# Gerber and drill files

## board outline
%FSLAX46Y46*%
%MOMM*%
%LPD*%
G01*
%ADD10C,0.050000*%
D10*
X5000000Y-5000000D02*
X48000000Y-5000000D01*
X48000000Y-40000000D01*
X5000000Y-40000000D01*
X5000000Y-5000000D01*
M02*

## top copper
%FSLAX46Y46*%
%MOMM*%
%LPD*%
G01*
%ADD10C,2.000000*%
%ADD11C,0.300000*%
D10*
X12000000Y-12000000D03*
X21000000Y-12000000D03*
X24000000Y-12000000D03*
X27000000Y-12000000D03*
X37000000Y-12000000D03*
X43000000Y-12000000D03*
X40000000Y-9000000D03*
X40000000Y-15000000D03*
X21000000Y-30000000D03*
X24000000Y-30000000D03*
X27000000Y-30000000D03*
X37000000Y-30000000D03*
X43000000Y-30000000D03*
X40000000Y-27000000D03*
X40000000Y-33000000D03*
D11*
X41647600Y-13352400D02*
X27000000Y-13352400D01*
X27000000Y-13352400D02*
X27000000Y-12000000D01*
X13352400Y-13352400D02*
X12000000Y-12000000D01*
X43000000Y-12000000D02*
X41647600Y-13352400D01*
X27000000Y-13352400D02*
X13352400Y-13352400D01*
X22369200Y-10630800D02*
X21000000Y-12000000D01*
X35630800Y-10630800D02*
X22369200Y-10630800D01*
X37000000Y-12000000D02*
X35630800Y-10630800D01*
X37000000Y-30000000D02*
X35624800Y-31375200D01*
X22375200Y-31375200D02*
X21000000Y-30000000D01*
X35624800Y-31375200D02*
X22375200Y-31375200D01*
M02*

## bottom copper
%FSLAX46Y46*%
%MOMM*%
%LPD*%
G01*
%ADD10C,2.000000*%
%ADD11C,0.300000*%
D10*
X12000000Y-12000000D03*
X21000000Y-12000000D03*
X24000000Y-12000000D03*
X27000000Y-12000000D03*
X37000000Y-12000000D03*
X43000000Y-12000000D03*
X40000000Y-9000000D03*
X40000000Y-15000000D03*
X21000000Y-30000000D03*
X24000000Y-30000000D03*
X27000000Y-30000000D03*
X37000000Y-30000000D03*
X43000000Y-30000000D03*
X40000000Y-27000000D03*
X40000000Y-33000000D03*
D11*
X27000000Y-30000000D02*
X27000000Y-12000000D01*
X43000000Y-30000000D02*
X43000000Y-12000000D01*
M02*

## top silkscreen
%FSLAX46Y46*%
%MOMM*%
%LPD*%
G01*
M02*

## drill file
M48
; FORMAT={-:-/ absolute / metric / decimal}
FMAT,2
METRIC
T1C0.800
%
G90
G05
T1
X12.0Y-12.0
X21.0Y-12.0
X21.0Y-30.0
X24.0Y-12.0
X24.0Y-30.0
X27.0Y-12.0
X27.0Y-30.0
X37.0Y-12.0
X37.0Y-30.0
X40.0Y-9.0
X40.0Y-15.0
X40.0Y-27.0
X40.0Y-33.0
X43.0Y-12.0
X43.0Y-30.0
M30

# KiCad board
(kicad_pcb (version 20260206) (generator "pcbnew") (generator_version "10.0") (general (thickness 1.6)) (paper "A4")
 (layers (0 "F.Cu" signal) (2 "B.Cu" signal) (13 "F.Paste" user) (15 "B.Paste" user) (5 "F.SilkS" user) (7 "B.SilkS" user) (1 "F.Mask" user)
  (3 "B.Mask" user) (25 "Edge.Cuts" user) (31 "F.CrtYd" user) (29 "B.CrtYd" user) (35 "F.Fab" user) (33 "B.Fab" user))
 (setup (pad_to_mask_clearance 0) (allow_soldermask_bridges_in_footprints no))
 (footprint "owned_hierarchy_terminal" (layer "F.Cu") (at 12 12)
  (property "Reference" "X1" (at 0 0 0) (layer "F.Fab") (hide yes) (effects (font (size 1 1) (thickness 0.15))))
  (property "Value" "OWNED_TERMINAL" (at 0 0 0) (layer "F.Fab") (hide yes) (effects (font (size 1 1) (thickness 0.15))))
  (pad "1" thru_hole circle (at 0 0) (size 2 2) (drill 0.8) (layers "*.Cu" "*.Mask") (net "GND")))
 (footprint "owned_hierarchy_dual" (layer "F.Cu") (at 24 12)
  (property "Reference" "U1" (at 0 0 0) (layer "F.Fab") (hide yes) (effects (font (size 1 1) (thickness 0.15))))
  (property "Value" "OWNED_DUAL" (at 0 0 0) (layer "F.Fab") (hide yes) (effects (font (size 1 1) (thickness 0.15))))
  (pad "1" thru_hole circle (at -3 0) (size 2 2) (drill 0.8) (layers "*.Cu" "*.Mask") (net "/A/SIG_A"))
  (pad "2" thru_hole circle (at 0 0) (size 2 2) (drill 0.8) (layers "*.Cu" "*.Mask") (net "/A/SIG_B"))
  (pad "3" thru_hole circle (at 3 0) (size 2 2) (drill 0.8) (layers "*.Cu" "*.Mask") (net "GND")))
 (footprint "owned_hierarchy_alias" (layer "F.Cu") (at 40 12)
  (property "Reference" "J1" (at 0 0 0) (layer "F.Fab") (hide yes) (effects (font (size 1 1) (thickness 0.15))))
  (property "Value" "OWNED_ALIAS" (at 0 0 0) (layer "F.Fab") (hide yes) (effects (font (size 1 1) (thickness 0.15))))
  (pad "R" thru_hole circle (at -3 0) (size 2 2) (drill 0.8) (layers "*.Cu" "*.Mask") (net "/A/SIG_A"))
  (pad "T" thru_hole circle (at 3 0) (size 2 2) (drill 0.8) (layers "*.Cu" "*.Mask") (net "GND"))
  (pad "MP" thru_hole circle (at 0 -3) (size 2 2) (drill 0.8) (layers "*.Cu" "*.Mask"))
  (pad "MP" thru_hole circle (at 0 3) (size 2 2) (drill 0.8) (layers "*.Cu" "*.Mask")))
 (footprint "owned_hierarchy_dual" (layer "F.Cu") (at 24 30)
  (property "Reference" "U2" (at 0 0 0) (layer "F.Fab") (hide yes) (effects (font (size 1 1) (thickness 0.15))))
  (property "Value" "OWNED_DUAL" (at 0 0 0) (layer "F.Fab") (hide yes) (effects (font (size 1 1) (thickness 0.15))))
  (pad "1" thru_hole circle (at -3 0) (size 2 2) (drill 0.8) (layers "*.Cu" "*.Mask") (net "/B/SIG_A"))
  (pad "2" thru_hole circle (at 0 0) (size 2 2) (drill 0.8) (layers "*.Cu" "*.Mask") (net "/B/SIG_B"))
  (pad "3" thru_hole circle (at 3 0) (size 2 2) (drill 0.8) (layers "*.Cu" "*.Mask") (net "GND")))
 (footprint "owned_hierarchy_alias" (layer "F.Cu") (at 40 30)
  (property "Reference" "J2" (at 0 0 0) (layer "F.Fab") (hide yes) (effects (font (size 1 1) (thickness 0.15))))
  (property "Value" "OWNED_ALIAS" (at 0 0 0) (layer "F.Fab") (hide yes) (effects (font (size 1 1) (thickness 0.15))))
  (pad "R" thru_hole circle (at -3 0) (size 2 2) (drill 0.8) (layers "*.Cu" "*.Mask") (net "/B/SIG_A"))
  (pad "T" thru_hole circle (at 3 0) (size 2 2) (drill 0.8) (layers "*.Cu" "*.Mask") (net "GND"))
  (pad "MP" thru_hole circle (at 0 -3) (size 2 2) (drill 0.8) (layers "*.Cu" "*.Mask"))
  (pad "MP" thru_hole circle (at 0 3) (size 2 2) (drill 0.8) (layers "*.Cu" "*.Mask")))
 (gr_rect (start 5 5) (end 48 40) (stroke (width 0.05) (type default)) (fill none) (layer "Edge.Cuts"))
 (segment (start 41.6476 13.3524) (end 27 13.3524) (width 0.3) (layer "F.Cu") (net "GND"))
 (segment (start 27 13.3524) (end 27 12) (width 0.3) (layer "F.Cu") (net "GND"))
 (segment (start 13.3524 13.3524) (end 12 12) (width 0.3) (layer "F.Cu") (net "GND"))
 (segment (start 43 12) (end 41.6476 13.3524) (width 0.3) (layer "F.Cu") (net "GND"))
 (segment (start 27 13.3524) (end 13.3524 13.3524) (width 0.3) (layer "F.Cu") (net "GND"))
 (segment (start 27 30) (end 27 12) (width 0.3) (layer "B.Cu") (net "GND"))
 (segment (start 43 30) (end 43 12) (width 0.3) (layer "B.Cu") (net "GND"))
 (segment (start 22.3692 10.6308) (end 21 12) (width 0.3) (layer "F.Cu") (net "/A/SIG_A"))
 (segment (start 35.6308 10.6308) (end 22.3692 10.6308) (width 0.3) (layer "F.Cu") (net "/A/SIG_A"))
 (segment (start 37 12) (end 35.6308 10.6308) (width 0.3) (layer "F.Cu") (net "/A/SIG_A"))
 (segment (start 37 30) (end 35.6248 31.3752) (width 0.3) (layer "F.Cu") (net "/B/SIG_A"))
 (segment (start 22.3752 31.3752) (end 21 30) (width 0.3) (layer "F.Cu") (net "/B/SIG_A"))
 (segment (start 35.6248 31.3752) (end 22.3752 31.3752) (width 0.3) (layer "F.Cu") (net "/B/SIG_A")))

